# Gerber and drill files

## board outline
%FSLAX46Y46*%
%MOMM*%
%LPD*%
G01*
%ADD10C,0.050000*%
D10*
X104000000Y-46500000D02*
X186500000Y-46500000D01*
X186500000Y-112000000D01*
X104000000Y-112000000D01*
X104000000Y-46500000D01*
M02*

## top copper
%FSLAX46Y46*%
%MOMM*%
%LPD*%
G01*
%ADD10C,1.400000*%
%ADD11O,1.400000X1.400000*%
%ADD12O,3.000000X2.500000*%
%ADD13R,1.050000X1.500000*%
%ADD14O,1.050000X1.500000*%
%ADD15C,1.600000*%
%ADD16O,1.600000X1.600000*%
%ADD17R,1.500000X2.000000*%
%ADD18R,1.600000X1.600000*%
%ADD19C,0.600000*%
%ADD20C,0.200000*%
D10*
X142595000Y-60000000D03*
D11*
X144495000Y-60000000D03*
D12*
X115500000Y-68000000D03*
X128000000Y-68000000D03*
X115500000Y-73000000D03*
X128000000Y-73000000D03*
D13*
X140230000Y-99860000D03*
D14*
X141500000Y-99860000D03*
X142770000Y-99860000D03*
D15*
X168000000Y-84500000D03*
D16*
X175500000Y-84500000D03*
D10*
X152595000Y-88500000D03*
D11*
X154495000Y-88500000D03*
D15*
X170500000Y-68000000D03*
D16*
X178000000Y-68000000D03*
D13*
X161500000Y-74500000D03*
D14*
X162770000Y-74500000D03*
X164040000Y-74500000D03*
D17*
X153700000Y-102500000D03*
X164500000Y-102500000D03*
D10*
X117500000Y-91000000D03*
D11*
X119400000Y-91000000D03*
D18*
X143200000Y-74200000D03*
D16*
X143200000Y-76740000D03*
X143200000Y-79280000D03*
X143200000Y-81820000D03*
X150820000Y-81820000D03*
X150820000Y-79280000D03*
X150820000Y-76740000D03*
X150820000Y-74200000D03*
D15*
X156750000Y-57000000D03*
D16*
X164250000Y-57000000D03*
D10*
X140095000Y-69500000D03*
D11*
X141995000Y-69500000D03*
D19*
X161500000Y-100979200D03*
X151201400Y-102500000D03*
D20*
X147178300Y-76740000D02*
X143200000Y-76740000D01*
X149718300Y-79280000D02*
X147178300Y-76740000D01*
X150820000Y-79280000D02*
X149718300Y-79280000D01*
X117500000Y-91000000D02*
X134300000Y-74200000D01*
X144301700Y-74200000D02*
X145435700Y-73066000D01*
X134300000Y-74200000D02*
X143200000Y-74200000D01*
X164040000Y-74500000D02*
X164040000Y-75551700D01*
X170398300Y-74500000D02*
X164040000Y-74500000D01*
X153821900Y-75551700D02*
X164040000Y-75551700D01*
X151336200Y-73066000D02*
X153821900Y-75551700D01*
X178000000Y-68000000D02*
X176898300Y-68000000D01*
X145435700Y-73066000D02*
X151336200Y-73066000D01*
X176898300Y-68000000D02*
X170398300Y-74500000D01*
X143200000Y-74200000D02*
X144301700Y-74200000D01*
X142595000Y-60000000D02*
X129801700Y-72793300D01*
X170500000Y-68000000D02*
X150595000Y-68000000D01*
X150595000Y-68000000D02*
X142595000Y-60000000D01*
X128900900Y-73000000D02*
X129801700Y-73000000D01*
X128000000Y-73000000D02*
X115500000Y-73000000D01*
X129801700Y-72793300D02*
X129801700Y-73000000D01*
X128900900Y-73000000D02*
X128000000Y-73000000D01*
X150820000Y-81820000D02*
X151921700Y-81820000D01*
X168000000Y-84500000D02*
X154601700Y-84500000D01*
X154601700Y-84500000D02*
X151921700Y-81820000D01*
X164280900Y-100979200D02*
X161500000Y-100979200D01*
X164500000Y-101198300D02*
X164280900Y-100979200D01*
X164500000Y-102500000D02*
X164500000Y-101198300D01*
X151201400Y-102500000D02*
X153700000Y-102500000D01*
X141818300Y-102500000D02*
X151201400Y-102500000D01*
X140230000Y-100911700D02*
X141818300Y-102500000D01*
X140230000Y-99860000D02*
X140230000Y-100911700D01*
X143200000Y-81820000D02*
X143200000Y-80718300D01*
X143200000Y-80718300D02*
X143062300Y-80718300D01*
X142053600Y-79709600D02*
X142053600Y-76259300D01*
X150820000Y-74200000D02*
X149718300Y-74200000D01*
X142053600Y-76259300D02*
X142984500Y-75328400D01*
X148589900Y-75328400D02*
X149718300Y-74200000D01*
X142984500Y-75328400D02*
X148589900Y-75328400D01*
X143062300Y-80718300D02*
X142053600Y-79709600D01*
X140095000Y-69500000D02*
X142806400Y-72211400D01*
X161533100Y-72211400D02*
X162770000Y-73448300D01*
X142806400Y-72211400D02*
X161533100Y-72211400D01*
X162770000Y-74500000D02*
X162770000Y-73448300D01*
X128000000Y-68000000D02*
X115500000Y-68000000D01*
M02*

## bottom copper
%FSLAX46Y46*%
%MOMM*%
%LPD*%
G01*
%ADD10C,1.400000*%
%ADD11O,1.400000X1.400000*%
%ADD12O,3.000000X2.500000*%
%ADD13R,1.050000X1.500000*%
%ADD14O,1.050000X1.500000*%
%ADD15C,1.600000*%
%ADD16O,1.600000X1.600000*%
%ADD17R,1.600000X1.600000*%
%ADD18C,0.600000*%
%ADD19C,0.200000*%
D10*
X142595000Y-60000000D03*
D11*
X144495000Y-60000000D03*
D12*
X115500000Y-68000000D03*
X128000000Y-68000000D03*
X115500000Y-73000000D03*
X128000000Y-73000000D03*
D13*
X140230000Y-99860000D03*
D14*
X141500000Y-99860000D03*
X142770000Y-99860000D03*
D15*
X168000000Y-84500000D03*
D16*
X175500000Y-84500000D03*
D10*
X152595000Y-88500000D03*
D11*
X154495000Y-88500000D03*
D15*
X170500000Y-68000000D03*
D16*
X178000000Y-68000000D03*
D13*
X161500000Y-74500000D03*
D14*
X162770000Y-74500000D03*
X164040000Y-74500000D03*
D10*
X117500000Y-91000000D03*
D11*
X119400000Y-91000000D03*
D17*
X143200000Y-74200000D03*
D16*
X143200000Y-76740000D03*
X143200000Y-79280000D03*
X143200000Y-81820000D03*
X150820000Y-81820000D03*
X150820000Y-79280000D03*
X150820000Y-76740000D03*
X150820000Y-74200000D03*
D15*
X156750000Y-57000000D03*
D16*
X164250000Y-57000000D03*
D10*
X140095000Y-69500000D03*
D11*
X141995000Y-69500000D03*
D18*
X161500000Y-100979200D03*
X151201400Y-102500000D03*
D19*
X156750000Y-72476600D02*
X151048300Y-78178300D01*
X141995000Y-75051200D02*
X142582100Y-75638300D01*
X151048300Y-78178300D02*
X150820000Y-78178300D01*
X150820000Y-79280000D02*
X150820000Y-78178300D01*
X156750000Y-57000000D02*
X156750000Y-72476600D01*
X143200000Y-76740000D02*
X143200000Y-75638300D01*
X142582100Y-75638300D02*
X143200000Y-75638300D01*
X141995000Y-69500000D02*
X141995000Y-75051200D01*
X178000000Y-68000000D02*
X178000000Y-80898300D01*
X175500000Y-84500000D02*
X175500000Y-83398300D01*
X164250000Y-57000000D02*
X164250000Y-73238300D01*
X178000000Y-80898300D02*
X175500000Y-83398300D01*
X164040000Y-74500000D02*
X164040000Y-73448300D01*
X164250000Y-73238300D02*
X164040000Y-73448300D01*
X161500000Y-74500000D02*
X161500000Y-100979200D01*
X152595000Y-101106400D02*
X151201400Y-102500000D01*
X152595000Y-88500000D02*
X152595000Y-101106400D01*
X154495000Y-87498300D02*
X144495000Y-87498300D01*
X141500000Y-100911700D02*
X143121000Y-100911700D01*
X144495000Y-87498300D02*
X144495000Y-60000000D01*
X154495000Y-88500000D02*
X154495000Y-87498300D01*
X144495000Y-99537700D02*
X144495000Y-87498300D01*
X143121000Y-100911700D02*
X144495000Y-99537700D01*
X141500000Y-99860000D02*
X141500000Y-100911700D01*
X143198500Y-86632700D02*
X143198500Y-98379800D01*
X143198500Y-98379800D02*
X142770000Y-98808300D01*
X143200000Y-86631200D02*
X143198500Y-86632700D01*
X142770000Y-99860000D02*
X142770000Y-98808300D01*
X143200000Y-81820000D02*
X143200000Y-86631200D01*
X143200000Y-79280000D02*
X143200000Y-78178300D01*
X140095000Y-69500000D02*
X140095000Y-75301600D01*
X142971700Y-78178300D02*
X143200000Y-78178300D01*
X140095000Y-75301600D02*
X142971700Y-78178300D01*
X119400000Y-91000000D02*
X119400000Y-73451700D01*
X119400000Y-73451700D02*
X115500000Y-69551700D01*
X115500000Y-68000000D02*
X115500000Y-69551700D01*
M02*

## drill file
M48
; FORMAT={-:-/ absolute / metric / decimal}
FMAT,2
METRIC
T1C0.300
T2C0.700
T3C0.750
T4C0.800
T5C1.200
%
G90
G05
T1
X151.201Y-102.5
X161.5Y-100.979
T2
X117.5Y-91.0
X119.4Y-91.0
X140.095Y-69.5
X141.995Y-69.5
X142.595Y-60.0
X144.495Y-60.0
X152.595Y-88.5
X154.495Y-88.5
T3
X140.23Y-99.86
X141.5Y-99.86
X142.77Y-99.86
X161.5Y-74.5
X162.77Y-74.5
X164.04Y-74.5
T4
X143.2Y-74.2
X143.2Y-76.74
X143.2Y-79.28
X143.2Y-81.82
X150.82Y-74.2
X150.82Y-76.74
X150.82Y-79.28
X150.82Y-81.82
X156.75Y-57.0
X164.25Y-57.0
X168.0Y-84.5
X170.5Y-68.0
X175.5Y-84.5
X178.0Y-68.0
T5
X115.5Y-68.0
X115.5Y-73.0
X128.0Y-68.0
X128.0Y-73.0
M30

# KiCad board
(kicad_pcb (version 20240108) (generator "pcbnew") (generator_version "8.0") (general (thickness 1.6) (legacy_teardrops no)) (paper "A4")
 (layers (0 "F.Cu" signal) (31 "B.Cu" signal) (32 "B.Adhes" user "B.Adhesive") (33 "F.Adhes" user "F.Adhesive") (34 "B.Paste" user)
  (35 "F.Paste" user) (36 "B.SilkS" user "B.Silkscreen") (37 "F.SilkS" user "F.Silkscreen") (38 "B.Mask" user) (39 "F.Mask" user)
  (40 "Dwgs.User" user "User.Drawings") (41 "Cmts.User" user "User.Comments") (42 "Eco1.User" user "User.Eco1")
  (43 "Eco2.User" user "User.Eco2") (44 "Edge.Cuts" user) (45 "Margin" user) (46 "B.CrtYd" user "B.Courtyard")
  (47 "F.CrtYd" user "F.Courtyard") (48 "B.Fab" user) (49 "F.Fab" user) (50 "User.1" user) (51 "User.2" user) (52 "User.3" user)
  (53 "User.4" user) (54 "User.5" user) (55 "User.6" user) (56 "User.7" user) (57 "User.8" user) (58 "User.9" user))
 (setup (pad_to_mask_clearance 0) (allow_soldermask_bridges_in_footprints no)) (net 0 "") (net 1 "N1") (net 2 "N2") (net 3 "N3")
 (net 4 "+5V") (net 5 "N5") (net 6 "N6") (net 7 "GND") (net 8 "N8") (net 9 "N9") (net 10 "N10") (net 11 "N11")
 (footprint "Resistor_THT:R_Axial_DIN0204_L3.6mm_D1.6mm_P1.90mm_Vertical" (layer "F.Cu") (at 142.595 60)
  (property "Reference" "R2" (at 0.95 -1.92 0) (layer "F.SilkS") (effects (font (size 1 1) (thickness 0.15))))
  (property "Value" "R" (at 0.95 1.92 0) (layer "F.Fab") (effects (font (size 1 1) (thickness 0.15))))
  (pad "1" thru_hole circle (at 0 0) (size 1.4 1.4) (drill 0.7) (layers "*.Cu" "*.Mask") (remove_unused_layers no) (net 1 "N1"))
  (pad "2" thru_hole oval (at 1.9 0) (size 1.4 1.4) (drill 0.7) (layers "*.Cu" "*.Mask") (remove_unused_layers no) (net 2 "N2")))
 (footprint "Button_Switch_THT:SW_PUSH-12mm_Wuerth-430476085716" (layer "F.Cu") (at 115.5 68)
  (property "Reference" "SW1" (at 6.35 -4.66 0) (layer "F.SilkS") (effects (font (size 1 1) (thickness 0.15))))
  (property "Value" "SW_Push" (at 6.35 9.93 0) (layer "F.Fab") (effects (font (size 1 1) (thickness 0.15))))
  (pad "1" thru_hole oval (at 0 0) (size 3 2.5) (drill 1.2) (layers "*.Cu" "*.Mask") (remove_unused_layers no) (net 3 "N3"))
  (pad "1" thru_hole oval (at 12.5 0) (size 3 2.5) (drill 1.2) (layers "*.Cu" "*.Mask") (remove_unused_layers no) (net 3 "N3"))
  (pad "2" thru_hole oval (at 0 5) (size 3 2.5) (drill 1.2) (layers "*.Cu" "*.Mask") (remove_unused_layers no) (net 1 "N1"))
  (pad "2" thru_hole oval (at 12.5 5) (size 3 2.5) (drill 1.2) (layers "*.Cu" "*.Mask") (remove_unused_layers no) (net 1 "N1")))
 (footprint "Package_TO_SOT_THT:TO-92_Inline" (layer "F.Cu") (at 140.23 99.86)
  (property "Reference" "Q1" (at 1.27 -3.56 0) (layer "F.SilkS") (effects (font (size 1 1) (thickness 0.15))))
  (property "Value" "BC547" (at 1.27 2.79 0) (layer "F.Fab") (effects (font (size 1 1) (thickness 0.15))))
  (pad "1" thru_hole rect (at 0 0) (size 1.05 1.5) (drill 0.75) (layers "*.Cu" "*.Mask") (remove_unused_layers no) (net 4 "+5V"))
  (pad "2" thru_hole oval (at 1.27 0) (size 1.05 1.5) (drill 0.75) (layers "*.Cu" "*.Mask") (remove_unused_layers no) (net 2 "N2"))
  (pad "3" thru_hole oval (at 2.54 0) (size 1.05 1.5) (drill 0.75) (layers "*.Cu" "*.Mask") (remove_unused_layers no) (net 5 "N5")))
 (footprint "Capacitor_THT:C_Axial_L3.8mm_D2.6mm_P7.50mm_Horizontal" (layer "F.Cu") (at 168 84.5)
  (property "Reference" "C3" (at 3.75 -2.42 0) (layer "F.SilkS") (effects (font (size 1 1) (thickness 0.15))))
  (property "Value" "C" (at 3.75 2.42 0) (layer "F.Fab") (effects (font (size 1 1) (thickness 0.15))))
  (pad "1" thru_hole circle (at 0 0) (size 1.6 1.6) (drill 0.8) (layers "*.Cu" "*.Mask") (remove_unused_layers no) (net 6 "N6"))
  (pad "2" thru_hole oval (at 7.5 0) (size 1.6 1.6) (drill 0.8) (layers "*.Cu" "*.Mask") (remove_unused_layers no) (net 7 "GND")))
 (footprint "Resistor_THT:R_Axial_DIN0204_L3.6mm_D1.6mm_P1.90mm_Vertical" (layer "F.Cu") (at 152.595 88.5)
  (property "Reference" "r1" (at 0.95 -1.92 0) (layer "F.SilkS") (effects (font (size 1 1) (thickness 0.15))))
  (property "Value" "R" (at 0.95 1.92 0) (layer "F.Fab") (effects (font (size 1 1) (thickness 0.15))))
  (pad "1" thru_hole circle (at 0 0) (size 1.4 1.4) (drill 0.7) (layers "*.Cu" "*.Mask") (remove_unused_layers no) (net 4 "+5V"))
  (pad "2" thru_hole oval (at 1.9 0) (size 1.4 1.4) (drill 0.7) (layers "*.Cu" "*.Mask") (remove_unused_layers no) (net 2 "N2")))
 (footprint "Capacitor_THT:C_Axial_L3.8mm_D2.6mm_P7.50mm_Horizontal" (layer "F.Cu") (at 170.5 68)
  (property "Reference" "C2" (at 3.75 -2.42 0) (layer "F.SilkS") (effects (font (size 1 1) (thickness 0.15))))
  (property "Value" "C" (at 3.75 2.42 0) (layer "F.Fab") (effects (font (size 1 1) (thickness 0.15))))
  (pad "1" thru_hole circle (at 0 0) (size 1.6 1.6) (drill 0.8) (layers "*.Cu" "*.Mask") (remove_unused_layers no) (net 1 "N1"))
  (pad "2" thru_hole oval (at 7.5 0) (size 1.6 1.6) (drill 0.8) (layers "*.Cu" "*.Mask") (remove_unused_layers no) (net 7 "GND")))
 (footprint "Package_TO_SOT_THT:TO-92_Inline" (layer "F.Cu") (at 161.5 74.5)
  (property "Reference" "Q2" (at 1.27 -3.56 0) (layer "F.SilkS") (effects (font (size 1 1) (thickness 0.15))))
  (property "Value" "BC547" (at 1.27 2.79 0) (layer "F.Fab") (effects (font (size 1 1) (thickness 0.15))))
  (pad "1" thru_hole rect (at 0 0) (size 1.05 1.5) (drill 0.75) (layers "*.Cu" "*.Mask") (remove_unused_layers no) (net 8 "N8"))
  (pad "2" thru_hole oval (at 1.27 0) (size 1.05 1.5) (drill 0.75) (layers "*.Cu" "*.Mask") (remove_unused_layers no) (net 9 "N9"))
  (pad "3" thru_hole oval (at 2.54 0) (size 1.05 1.5) (drill 0.75) (layers "*.Cu" "*.Mask") (remove_unused_layers no) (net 7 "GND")))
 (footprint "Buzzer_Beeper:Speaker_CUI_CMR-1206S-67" (layer "F.Cu") (at 159.1 100.2)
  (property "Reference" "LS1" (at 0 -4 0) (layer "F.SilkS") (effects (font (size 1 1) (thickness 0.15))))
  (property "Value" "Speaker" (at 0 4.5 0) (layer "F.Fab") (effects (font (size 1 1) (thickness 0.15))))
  (pad "1" smd rect (at -5.4 2.3 180) (size 1.5 2) (layers "F.Cu" "F.Mask") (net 4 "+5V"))
  (pad "2" smd rect (at 5.4 2.3 180) (size 1.5 2) (layers "F.Cu" "F.Mask") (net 8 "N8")))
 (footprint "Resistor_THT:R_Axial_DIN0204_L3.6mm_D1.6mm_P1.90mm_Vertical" (layer "F.Cu") (at 117.5 91)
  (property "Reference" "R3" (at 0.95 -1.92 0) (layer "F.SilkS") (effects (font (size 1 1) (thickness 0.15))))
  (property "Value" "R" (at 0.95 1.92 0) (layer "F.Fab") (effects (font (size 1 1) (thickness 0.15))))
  (pad "1" thru_hole circle (at 0 0) (size 1.4 1.4) (drill 0.7) (layers "*.Cu" "*.Mask") (remove_unused_layers no) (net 7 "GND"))
  (pad "2" thru_hole oval (at 1.9 0) (size 1.4 1.4) (drill 0.7) (layers "*.Cu" "*.Mask") (remove_unused_layers no) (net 3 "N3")))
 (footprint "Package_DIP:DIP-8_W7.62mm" (layer "F.Cu") (at 143.2 74.2)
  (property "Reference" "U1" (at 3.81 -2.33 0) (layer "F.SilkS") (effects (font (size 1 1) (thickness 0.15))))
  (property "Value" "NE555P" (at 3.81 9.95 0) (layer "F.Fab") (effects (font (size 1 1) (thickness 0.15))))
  (pad "1" thru_hole rect (at 0 0) (size 1.6 1.6) (drill 0.8) (layers "*.Cu" "*.Mask") (remove_unused_layers no) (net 7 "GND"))
  (pad "2" thru_hole oval (at 0 2.54) (size 1.6 1.6) (drill 0.8) (layers "*.Cu" "*.Mask") (remove_unused_layers no) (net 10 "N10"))
  (pad "3" thru_hole oval (at 0 5.08) (size 1.6 1.6) (drill 0.8) (layers "*.Cu" "*.Mask") (remove_unused_layers no) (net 9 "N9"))
  (pad "4" thru_hole oval (at 0 7.62) (size 1.6 1.6) (drill 0.8) (layers "*.Cu" "*.Mask") (remove_unused_layers no) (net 5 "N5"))
  (pad "5" thru_hole oval (at 7.62 7.62) (size 1.6 1.6) (drill 0.8) (layers "*.Cu" "*.Mask") (remove_unused_layers no) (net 6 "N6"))
  (pad "6" thru_hole oval (at 7.62 5.08) (size 1.6 1.6) (drill 0.8) (layers "*.Cu" "*.Mask") (remove_unused_layers no) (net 10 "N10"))
  (pad "7" thru_hole oval (at 7.62 2.54) (size 1.6 1.6) (drill 0.8) (layers "*.Cu" "*.Mask") (remove_unused_layers no) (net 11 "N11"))
  (pad "8" thru_hole oval (at 7.62 0) (size 1.6 1.6) (drill 0.8) (layers "*.Cu" "*.Mask") (remove_unused_layers no) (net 5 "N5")))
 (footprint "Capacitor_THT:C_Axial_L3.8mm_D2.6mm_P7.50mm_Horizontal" (layer "F.Cu") (at 156.75 57)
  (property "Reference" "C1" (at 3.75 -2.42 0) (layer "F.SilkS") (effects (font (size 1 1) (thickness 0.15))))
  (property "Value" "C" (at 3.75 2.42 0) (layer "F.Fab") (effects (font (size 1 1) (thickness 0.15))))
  (pad "1" thru_hole circle (at 0 0) (size 1.6 1.6) (drill 0.8) (layers "*.Cu" "*.Mask") (remove_unused_layers no) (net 10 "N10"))
  (pad "2" thru_hole oval (at 7.5 0) (size 1.6 1.6) (drill 0.8) (layers "*.Cu" "*.Mask") (remove_unused_layers no) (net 7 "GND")))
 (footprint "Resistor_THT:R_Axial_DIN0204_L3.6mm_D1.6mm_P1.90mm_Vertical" (layer "F.Cu") (at 140.095 69.5)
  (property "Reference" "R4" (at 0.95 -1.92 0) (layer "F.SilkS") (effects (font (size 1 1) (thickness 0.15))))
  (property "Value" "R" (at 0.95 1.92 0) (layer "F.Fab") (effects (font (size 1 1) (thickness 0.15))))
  (pad "1" thru_hole circle (at 0 0) (size 1.4 1.4) (drill 0.7) (layers "*.Cu" "*.Mask") (remove_unused_layers no) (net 9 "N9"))
  (pad "2" thru_hole oval (at 1.9 0) (size 1.4 1.4) (drill 0.7) (layers "*.Cu" "*.Mask") (remove_unused_layers no) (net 10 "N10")))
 (gr_rect (start 104 46.5) (end 186.5 112) (stroke (width 0.05) (type default)) (fill none) (layer "Edge.Cuts"))
 (segment (start 147.1783 76.74) (end 143.2 76.74) (width 0.2) (layer "F.Cu") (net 10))
 (segment (start 149.7183 79.28) (end 147.1783 76.74) (width 0.2) (layer "F.Cu") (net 10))
 (segment (start 150.82 79.28) (end 149.7183 79.28) (width 0.2) (layer "F.Cu") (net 10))
 (segment (start 156.75 72.4766) (end 151.0483 78.1783) (width 0.2) (layer "B.Cu") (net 10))
 (segment (start 141.995 75.0512) (end 142.5821 75.6383) (width 0.2) (layer "B.Cu") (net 10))
 (segment (start 151.0483 78.1783) (end 150.82 78.1783) (width 0.2) (layer "B.Cu") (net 10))
 (segment (start 150.82 79.28) (end 150.82 78.1783) (width 0.2) (layer "B.Cu") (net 10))
 (segment (start 156.75 57) (end 156.75 72.4766) (width 0.2) (layer "B.Cu") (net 10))
 (segment (start 143.2 76.74) (end 143.2 75.6383) (width 0.2) (layer "B.Cu") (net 10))
 (segment (start 142.5821 75.6383) (end 143.2 75.6383) (width 0.2) (layer "B.Cu") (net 10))
 (segment (start 141.995 69.5) (end 141.995 75.0512) (width 0.2) (layer "B.Cu") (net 10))
 (segment (start 117.5 91) (end 134.3 74.2) (width 0.2) (layer "F.Cu") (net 7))
 (segment (start 144.3017 74.2) (end 145.4357 73.066) (width 0.2) (layer "F.Cu") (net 7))
 (segment (start 134.3 74.2) (end 143.2 74.2) (width 0.2) (layer "F.Cu") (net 7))
 (segment (start 164.04 74.5) (end 164.04 75.5517) (width 0.2) (layer "F.Cu") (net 7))
 (segment (start 170.3983 74.5) (end 164.04 74.5) (width 0.2) (layer "F.Cu") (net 7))
 (segment (start 153.8219 75.5517) (end 164.04 75.5517) (width 0.2) (layer "F.Cu") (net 7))
 (segment (start 151.3362 73.066) (end 153.8219 75.5517) (width 0.2) (layer "F.Cu") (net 7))
 (segment (start 178 68) (end 176.8983 68) (width 0.2) (layer "F.Cu") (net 7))
 (segment (start 145.4357 73.066) (end 151.3362 73.066) (width 0.2) (layer "F.Cu") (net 7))
 (segment (start 176.8983 68) (end 170.3983 74.5) (width 0.2) (layer "F.Cu") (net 7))
 (segment (start 143.2 74.2) (end 144.3017 74.2) (width 0.2) (layer "F.Cu") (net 7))
 (segment (start 178 68) (end 178 80.8983) (width 0.2) (layer "B.Cu") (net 7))
 (segment (start 175.5 84.5) (end 175.5 83.3983) (width 0.2) (layer "B.Cu") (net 7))
 (segment (start 164.25 57) (end 164.25 73.2383) (width 0.2) (layer "B.Cu") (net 7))
 (segment (start 178 80.8983) (end 175.5 83.3983) (width 0.2) (layer "B.Cu") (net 7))
 (segment (start 164.04 74.5) (end 164.04 73.4483) (width 0.2) (layer "B.Cu") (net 7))
 (segment (start 164.25 73.2383) (end 164.04 73.4483) (width 0.2) (layer "B.Cu") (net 7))
 (segment (start 142.595 60) (end 129.8017 72.7933) (width 0.2) (layer "F.Cu") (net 1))
 (segment (start 170.5 68) (end 150.595 68) (width 0.2) (layer "F.Cu") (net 1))
 (segment (start 150.595 68) (end 142.595 60) (width 0.2) (layer "F.Cu") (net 1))
 (segment (start 128.9009 73) (end 129.8017 73) (width 0.2) (layer "F.Cu") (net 1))
 (segment (start 128 73) (end 115.5 73) (width 0.2) (layer "F.Cu") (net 1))
 (segment (start 129.8017 72.7933) (end 129.8017 73) (width 0.2) (layer "F.Cu") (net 1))
 (segment (start 128.9009 73) (end 128 73) (width 0.2) (layer "F.Cu") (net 1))
 (segment (start 150.82 81.82) (end 151.9217 81.82) (width 0.2) (layer "F.Cu") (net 6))
 (segment (start 168 84.5) (end 154.6017 84.5) (width 0.2) (layer "F.Cu") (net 6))
 (segment (start 154.6017 84.5) (end 151.9217 81.82) (width 0.2) (layer "F.Cu") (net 6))
 (segment (start 164.2809 100.9792) (end 161.5 100.9792) (width 0.2) (layer "F.Cu") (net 8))
 (segment (start 164.5 101.1983) (end 164.2809 100.9792) (width 0.2) (layer "F.Cu") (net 8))
 (segment (start 164.5 102.5) (end 164.5 101.1983) (width 0.2) (layer "F.Cu") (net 8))
 (via (at 161.5 100.9792) (size 0.6) (drill 0.3) (layers "F.Cu" "B.Cu") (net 8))
 (segment (start 161.5 74.5) (end 161.5 100.9792) (width 0.2) (layer "B.Cu") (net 8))
 (segment (start 151.2014 102.5) (end 153.7 102.5) (width 0.2) (layer "F.Cu") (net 4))
 (segment (start 141.8183 102.5) (end 151.2014 102.5) (width 0.2) (layer "F.Cu") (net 4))
 (segment (start 140.23 100.9117) (end 141.8183 102.5) (width 0.2) (layer "F.Cu") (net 4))
 (segment (start 140.23 99.86) (end 140.23 100.9117) (width 0.2) (layer "F.Cu") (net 4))
 (via (at 151.2014 102.5) (size 0.6) (drill 0.3) (layers "F.Cu" "B.Cu") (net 4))
 (segment (start 152.595 101.1064) (end 151.2014 102.5) (width 0.2) (layer "B.Cu") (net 4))
 (segment (start 152.595 88.5) (end 152.595 101.1064) (width 0.2) (layer "B.Cu") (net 4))
 (segment (start 154.495 87.4983) (end 144.495 87.4983) (width 0.2) (layer "B.Cu") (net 2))
 (segment (start 141.5 100.9117) (end 143.121 100.9117) (width 0.2) (layer "B.Cu") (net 2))
 (segment (start 144.495 87.4983) (end 144.495 60) (width 0.2) (layer "B.Cu") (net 2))
 (segment (start 154.495 88.5) (end 154.495 87.4983) (width 0.2) (layer "B.Cu") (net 2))
 (segment (start 144.495 99.5377) (end 144.495 87.4983) (width 0.2) (layer "B.Cu") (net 2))
 (segment (start 143.121 100.9117) (end 144.495 99.5377) (width 0.2) (layer "B.Cu") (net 2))
 (segment (start 141.5 99.86) (end 141.5 100.9117) (width 0.2) (layer "B.Cu") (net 2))
 (segment (start 143.2 81.82) (end 143.2 80.7183) (width 0.2) (layer "F.Cu") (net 5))
 (segment (start 143.2 80.7183) (end 143.0623 80.7183) (width 0.2) (layer "F.Cu") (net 5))
 (segment (start 142.0536 79.7096) (end 142.0536 76.2593) (width 0.2) (layer "F.Cu") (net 5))
 (segment (start 150.82 74.2) (end 149.7183 74.2) (width 0.2) (layer "F.Cu") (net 5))
 (segment (start 142.0536 76.2593) (end 142.9845 75.3284) (width 0.2) (layer "F.Cu") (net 5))
 (segment (start 148.5899 75.3284) (end 149.7183 74.2) (width 0.2) (layer "F.Cu") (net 5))
 (segment (start 142.9845 75.3284) (end 148.5899 75.3284) (width 0.2) (layer "F.Cu") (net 5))
 (segment (start 143.0623 80.7183) (end 142.0536 79.7096) (width 0.2) (layer "F.Cu") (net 5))
 (segment (start 143.1985 86.6327) (end 143.1985 98.3798) (width 0.2) (layer "B.Cu") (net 5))
 (segment (start 143.1985 98.3798) (end 142.77 98.8083) (width 0.2) (layer "B.Cu") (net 5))
 (segment (start 143.2 86.6312) (end 143.1985 86.6327) (width 0.2) (layer "B.Cu") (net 5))
 (segment (start 142.77 99.86) (end 142.77 98.8083) (width 0.2) (layer "B.Cu") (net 5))
 (segment (start 143.2 81.82) (end 143.2 86.6312) (width 0.2) (layer "B.Cu") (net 5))
 (segment (start 140.095 69.5) (end 142.8064 72.2114) (width 0.2) (layer "F.Cu") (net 9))
 (segment (start 161.5331 72.2114) (end 162.77 73.4483) (width 0.2) (layer "F.Cu") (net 9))
 (segment (start 142.8064 72.2114) (end 161.5331 72.2114) (width 0.2) (layer "F.Cu") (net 9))
 (segment (start 162.77 74.5) (end 162.77 73.4483) (width 0.2) (layer "F.Cu") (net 9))
 (segment (start 143.2 79.28) (end 143.2 78.1783) (width 0.2) (layer "B.Cu") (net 9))
 (segment (start 140.095 69.5) (end 140.095 75.3016) (width 0.2) (layer "B.Cu") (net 9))
 (segment (start 142.9717 78.1783) (end 143.2 78.1783) (width 0.2) (layer "B.Cu") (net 9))
 (segment (start 140.095 75.3016) (end 142.9717 78.1783) (width 0.2) (layer "B.Cu") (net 9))
 (segment (start 128 68) (end 115.5 68) (width 0.2) (layer "F.Cu") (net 3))
 (segment (start 119.4 91) (end 119.4 73.4517) (width 0.2) (layer "B.Cu") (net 3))
 (segment (start 119.4 73.4517) (end 115.5 69.5517) (width 0.2) (layer "B.Cu") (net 3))
 (segment (start 115.5 68) (end 115.5 69.5517) (width 0.2) (layer "B.Cu") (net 3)))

